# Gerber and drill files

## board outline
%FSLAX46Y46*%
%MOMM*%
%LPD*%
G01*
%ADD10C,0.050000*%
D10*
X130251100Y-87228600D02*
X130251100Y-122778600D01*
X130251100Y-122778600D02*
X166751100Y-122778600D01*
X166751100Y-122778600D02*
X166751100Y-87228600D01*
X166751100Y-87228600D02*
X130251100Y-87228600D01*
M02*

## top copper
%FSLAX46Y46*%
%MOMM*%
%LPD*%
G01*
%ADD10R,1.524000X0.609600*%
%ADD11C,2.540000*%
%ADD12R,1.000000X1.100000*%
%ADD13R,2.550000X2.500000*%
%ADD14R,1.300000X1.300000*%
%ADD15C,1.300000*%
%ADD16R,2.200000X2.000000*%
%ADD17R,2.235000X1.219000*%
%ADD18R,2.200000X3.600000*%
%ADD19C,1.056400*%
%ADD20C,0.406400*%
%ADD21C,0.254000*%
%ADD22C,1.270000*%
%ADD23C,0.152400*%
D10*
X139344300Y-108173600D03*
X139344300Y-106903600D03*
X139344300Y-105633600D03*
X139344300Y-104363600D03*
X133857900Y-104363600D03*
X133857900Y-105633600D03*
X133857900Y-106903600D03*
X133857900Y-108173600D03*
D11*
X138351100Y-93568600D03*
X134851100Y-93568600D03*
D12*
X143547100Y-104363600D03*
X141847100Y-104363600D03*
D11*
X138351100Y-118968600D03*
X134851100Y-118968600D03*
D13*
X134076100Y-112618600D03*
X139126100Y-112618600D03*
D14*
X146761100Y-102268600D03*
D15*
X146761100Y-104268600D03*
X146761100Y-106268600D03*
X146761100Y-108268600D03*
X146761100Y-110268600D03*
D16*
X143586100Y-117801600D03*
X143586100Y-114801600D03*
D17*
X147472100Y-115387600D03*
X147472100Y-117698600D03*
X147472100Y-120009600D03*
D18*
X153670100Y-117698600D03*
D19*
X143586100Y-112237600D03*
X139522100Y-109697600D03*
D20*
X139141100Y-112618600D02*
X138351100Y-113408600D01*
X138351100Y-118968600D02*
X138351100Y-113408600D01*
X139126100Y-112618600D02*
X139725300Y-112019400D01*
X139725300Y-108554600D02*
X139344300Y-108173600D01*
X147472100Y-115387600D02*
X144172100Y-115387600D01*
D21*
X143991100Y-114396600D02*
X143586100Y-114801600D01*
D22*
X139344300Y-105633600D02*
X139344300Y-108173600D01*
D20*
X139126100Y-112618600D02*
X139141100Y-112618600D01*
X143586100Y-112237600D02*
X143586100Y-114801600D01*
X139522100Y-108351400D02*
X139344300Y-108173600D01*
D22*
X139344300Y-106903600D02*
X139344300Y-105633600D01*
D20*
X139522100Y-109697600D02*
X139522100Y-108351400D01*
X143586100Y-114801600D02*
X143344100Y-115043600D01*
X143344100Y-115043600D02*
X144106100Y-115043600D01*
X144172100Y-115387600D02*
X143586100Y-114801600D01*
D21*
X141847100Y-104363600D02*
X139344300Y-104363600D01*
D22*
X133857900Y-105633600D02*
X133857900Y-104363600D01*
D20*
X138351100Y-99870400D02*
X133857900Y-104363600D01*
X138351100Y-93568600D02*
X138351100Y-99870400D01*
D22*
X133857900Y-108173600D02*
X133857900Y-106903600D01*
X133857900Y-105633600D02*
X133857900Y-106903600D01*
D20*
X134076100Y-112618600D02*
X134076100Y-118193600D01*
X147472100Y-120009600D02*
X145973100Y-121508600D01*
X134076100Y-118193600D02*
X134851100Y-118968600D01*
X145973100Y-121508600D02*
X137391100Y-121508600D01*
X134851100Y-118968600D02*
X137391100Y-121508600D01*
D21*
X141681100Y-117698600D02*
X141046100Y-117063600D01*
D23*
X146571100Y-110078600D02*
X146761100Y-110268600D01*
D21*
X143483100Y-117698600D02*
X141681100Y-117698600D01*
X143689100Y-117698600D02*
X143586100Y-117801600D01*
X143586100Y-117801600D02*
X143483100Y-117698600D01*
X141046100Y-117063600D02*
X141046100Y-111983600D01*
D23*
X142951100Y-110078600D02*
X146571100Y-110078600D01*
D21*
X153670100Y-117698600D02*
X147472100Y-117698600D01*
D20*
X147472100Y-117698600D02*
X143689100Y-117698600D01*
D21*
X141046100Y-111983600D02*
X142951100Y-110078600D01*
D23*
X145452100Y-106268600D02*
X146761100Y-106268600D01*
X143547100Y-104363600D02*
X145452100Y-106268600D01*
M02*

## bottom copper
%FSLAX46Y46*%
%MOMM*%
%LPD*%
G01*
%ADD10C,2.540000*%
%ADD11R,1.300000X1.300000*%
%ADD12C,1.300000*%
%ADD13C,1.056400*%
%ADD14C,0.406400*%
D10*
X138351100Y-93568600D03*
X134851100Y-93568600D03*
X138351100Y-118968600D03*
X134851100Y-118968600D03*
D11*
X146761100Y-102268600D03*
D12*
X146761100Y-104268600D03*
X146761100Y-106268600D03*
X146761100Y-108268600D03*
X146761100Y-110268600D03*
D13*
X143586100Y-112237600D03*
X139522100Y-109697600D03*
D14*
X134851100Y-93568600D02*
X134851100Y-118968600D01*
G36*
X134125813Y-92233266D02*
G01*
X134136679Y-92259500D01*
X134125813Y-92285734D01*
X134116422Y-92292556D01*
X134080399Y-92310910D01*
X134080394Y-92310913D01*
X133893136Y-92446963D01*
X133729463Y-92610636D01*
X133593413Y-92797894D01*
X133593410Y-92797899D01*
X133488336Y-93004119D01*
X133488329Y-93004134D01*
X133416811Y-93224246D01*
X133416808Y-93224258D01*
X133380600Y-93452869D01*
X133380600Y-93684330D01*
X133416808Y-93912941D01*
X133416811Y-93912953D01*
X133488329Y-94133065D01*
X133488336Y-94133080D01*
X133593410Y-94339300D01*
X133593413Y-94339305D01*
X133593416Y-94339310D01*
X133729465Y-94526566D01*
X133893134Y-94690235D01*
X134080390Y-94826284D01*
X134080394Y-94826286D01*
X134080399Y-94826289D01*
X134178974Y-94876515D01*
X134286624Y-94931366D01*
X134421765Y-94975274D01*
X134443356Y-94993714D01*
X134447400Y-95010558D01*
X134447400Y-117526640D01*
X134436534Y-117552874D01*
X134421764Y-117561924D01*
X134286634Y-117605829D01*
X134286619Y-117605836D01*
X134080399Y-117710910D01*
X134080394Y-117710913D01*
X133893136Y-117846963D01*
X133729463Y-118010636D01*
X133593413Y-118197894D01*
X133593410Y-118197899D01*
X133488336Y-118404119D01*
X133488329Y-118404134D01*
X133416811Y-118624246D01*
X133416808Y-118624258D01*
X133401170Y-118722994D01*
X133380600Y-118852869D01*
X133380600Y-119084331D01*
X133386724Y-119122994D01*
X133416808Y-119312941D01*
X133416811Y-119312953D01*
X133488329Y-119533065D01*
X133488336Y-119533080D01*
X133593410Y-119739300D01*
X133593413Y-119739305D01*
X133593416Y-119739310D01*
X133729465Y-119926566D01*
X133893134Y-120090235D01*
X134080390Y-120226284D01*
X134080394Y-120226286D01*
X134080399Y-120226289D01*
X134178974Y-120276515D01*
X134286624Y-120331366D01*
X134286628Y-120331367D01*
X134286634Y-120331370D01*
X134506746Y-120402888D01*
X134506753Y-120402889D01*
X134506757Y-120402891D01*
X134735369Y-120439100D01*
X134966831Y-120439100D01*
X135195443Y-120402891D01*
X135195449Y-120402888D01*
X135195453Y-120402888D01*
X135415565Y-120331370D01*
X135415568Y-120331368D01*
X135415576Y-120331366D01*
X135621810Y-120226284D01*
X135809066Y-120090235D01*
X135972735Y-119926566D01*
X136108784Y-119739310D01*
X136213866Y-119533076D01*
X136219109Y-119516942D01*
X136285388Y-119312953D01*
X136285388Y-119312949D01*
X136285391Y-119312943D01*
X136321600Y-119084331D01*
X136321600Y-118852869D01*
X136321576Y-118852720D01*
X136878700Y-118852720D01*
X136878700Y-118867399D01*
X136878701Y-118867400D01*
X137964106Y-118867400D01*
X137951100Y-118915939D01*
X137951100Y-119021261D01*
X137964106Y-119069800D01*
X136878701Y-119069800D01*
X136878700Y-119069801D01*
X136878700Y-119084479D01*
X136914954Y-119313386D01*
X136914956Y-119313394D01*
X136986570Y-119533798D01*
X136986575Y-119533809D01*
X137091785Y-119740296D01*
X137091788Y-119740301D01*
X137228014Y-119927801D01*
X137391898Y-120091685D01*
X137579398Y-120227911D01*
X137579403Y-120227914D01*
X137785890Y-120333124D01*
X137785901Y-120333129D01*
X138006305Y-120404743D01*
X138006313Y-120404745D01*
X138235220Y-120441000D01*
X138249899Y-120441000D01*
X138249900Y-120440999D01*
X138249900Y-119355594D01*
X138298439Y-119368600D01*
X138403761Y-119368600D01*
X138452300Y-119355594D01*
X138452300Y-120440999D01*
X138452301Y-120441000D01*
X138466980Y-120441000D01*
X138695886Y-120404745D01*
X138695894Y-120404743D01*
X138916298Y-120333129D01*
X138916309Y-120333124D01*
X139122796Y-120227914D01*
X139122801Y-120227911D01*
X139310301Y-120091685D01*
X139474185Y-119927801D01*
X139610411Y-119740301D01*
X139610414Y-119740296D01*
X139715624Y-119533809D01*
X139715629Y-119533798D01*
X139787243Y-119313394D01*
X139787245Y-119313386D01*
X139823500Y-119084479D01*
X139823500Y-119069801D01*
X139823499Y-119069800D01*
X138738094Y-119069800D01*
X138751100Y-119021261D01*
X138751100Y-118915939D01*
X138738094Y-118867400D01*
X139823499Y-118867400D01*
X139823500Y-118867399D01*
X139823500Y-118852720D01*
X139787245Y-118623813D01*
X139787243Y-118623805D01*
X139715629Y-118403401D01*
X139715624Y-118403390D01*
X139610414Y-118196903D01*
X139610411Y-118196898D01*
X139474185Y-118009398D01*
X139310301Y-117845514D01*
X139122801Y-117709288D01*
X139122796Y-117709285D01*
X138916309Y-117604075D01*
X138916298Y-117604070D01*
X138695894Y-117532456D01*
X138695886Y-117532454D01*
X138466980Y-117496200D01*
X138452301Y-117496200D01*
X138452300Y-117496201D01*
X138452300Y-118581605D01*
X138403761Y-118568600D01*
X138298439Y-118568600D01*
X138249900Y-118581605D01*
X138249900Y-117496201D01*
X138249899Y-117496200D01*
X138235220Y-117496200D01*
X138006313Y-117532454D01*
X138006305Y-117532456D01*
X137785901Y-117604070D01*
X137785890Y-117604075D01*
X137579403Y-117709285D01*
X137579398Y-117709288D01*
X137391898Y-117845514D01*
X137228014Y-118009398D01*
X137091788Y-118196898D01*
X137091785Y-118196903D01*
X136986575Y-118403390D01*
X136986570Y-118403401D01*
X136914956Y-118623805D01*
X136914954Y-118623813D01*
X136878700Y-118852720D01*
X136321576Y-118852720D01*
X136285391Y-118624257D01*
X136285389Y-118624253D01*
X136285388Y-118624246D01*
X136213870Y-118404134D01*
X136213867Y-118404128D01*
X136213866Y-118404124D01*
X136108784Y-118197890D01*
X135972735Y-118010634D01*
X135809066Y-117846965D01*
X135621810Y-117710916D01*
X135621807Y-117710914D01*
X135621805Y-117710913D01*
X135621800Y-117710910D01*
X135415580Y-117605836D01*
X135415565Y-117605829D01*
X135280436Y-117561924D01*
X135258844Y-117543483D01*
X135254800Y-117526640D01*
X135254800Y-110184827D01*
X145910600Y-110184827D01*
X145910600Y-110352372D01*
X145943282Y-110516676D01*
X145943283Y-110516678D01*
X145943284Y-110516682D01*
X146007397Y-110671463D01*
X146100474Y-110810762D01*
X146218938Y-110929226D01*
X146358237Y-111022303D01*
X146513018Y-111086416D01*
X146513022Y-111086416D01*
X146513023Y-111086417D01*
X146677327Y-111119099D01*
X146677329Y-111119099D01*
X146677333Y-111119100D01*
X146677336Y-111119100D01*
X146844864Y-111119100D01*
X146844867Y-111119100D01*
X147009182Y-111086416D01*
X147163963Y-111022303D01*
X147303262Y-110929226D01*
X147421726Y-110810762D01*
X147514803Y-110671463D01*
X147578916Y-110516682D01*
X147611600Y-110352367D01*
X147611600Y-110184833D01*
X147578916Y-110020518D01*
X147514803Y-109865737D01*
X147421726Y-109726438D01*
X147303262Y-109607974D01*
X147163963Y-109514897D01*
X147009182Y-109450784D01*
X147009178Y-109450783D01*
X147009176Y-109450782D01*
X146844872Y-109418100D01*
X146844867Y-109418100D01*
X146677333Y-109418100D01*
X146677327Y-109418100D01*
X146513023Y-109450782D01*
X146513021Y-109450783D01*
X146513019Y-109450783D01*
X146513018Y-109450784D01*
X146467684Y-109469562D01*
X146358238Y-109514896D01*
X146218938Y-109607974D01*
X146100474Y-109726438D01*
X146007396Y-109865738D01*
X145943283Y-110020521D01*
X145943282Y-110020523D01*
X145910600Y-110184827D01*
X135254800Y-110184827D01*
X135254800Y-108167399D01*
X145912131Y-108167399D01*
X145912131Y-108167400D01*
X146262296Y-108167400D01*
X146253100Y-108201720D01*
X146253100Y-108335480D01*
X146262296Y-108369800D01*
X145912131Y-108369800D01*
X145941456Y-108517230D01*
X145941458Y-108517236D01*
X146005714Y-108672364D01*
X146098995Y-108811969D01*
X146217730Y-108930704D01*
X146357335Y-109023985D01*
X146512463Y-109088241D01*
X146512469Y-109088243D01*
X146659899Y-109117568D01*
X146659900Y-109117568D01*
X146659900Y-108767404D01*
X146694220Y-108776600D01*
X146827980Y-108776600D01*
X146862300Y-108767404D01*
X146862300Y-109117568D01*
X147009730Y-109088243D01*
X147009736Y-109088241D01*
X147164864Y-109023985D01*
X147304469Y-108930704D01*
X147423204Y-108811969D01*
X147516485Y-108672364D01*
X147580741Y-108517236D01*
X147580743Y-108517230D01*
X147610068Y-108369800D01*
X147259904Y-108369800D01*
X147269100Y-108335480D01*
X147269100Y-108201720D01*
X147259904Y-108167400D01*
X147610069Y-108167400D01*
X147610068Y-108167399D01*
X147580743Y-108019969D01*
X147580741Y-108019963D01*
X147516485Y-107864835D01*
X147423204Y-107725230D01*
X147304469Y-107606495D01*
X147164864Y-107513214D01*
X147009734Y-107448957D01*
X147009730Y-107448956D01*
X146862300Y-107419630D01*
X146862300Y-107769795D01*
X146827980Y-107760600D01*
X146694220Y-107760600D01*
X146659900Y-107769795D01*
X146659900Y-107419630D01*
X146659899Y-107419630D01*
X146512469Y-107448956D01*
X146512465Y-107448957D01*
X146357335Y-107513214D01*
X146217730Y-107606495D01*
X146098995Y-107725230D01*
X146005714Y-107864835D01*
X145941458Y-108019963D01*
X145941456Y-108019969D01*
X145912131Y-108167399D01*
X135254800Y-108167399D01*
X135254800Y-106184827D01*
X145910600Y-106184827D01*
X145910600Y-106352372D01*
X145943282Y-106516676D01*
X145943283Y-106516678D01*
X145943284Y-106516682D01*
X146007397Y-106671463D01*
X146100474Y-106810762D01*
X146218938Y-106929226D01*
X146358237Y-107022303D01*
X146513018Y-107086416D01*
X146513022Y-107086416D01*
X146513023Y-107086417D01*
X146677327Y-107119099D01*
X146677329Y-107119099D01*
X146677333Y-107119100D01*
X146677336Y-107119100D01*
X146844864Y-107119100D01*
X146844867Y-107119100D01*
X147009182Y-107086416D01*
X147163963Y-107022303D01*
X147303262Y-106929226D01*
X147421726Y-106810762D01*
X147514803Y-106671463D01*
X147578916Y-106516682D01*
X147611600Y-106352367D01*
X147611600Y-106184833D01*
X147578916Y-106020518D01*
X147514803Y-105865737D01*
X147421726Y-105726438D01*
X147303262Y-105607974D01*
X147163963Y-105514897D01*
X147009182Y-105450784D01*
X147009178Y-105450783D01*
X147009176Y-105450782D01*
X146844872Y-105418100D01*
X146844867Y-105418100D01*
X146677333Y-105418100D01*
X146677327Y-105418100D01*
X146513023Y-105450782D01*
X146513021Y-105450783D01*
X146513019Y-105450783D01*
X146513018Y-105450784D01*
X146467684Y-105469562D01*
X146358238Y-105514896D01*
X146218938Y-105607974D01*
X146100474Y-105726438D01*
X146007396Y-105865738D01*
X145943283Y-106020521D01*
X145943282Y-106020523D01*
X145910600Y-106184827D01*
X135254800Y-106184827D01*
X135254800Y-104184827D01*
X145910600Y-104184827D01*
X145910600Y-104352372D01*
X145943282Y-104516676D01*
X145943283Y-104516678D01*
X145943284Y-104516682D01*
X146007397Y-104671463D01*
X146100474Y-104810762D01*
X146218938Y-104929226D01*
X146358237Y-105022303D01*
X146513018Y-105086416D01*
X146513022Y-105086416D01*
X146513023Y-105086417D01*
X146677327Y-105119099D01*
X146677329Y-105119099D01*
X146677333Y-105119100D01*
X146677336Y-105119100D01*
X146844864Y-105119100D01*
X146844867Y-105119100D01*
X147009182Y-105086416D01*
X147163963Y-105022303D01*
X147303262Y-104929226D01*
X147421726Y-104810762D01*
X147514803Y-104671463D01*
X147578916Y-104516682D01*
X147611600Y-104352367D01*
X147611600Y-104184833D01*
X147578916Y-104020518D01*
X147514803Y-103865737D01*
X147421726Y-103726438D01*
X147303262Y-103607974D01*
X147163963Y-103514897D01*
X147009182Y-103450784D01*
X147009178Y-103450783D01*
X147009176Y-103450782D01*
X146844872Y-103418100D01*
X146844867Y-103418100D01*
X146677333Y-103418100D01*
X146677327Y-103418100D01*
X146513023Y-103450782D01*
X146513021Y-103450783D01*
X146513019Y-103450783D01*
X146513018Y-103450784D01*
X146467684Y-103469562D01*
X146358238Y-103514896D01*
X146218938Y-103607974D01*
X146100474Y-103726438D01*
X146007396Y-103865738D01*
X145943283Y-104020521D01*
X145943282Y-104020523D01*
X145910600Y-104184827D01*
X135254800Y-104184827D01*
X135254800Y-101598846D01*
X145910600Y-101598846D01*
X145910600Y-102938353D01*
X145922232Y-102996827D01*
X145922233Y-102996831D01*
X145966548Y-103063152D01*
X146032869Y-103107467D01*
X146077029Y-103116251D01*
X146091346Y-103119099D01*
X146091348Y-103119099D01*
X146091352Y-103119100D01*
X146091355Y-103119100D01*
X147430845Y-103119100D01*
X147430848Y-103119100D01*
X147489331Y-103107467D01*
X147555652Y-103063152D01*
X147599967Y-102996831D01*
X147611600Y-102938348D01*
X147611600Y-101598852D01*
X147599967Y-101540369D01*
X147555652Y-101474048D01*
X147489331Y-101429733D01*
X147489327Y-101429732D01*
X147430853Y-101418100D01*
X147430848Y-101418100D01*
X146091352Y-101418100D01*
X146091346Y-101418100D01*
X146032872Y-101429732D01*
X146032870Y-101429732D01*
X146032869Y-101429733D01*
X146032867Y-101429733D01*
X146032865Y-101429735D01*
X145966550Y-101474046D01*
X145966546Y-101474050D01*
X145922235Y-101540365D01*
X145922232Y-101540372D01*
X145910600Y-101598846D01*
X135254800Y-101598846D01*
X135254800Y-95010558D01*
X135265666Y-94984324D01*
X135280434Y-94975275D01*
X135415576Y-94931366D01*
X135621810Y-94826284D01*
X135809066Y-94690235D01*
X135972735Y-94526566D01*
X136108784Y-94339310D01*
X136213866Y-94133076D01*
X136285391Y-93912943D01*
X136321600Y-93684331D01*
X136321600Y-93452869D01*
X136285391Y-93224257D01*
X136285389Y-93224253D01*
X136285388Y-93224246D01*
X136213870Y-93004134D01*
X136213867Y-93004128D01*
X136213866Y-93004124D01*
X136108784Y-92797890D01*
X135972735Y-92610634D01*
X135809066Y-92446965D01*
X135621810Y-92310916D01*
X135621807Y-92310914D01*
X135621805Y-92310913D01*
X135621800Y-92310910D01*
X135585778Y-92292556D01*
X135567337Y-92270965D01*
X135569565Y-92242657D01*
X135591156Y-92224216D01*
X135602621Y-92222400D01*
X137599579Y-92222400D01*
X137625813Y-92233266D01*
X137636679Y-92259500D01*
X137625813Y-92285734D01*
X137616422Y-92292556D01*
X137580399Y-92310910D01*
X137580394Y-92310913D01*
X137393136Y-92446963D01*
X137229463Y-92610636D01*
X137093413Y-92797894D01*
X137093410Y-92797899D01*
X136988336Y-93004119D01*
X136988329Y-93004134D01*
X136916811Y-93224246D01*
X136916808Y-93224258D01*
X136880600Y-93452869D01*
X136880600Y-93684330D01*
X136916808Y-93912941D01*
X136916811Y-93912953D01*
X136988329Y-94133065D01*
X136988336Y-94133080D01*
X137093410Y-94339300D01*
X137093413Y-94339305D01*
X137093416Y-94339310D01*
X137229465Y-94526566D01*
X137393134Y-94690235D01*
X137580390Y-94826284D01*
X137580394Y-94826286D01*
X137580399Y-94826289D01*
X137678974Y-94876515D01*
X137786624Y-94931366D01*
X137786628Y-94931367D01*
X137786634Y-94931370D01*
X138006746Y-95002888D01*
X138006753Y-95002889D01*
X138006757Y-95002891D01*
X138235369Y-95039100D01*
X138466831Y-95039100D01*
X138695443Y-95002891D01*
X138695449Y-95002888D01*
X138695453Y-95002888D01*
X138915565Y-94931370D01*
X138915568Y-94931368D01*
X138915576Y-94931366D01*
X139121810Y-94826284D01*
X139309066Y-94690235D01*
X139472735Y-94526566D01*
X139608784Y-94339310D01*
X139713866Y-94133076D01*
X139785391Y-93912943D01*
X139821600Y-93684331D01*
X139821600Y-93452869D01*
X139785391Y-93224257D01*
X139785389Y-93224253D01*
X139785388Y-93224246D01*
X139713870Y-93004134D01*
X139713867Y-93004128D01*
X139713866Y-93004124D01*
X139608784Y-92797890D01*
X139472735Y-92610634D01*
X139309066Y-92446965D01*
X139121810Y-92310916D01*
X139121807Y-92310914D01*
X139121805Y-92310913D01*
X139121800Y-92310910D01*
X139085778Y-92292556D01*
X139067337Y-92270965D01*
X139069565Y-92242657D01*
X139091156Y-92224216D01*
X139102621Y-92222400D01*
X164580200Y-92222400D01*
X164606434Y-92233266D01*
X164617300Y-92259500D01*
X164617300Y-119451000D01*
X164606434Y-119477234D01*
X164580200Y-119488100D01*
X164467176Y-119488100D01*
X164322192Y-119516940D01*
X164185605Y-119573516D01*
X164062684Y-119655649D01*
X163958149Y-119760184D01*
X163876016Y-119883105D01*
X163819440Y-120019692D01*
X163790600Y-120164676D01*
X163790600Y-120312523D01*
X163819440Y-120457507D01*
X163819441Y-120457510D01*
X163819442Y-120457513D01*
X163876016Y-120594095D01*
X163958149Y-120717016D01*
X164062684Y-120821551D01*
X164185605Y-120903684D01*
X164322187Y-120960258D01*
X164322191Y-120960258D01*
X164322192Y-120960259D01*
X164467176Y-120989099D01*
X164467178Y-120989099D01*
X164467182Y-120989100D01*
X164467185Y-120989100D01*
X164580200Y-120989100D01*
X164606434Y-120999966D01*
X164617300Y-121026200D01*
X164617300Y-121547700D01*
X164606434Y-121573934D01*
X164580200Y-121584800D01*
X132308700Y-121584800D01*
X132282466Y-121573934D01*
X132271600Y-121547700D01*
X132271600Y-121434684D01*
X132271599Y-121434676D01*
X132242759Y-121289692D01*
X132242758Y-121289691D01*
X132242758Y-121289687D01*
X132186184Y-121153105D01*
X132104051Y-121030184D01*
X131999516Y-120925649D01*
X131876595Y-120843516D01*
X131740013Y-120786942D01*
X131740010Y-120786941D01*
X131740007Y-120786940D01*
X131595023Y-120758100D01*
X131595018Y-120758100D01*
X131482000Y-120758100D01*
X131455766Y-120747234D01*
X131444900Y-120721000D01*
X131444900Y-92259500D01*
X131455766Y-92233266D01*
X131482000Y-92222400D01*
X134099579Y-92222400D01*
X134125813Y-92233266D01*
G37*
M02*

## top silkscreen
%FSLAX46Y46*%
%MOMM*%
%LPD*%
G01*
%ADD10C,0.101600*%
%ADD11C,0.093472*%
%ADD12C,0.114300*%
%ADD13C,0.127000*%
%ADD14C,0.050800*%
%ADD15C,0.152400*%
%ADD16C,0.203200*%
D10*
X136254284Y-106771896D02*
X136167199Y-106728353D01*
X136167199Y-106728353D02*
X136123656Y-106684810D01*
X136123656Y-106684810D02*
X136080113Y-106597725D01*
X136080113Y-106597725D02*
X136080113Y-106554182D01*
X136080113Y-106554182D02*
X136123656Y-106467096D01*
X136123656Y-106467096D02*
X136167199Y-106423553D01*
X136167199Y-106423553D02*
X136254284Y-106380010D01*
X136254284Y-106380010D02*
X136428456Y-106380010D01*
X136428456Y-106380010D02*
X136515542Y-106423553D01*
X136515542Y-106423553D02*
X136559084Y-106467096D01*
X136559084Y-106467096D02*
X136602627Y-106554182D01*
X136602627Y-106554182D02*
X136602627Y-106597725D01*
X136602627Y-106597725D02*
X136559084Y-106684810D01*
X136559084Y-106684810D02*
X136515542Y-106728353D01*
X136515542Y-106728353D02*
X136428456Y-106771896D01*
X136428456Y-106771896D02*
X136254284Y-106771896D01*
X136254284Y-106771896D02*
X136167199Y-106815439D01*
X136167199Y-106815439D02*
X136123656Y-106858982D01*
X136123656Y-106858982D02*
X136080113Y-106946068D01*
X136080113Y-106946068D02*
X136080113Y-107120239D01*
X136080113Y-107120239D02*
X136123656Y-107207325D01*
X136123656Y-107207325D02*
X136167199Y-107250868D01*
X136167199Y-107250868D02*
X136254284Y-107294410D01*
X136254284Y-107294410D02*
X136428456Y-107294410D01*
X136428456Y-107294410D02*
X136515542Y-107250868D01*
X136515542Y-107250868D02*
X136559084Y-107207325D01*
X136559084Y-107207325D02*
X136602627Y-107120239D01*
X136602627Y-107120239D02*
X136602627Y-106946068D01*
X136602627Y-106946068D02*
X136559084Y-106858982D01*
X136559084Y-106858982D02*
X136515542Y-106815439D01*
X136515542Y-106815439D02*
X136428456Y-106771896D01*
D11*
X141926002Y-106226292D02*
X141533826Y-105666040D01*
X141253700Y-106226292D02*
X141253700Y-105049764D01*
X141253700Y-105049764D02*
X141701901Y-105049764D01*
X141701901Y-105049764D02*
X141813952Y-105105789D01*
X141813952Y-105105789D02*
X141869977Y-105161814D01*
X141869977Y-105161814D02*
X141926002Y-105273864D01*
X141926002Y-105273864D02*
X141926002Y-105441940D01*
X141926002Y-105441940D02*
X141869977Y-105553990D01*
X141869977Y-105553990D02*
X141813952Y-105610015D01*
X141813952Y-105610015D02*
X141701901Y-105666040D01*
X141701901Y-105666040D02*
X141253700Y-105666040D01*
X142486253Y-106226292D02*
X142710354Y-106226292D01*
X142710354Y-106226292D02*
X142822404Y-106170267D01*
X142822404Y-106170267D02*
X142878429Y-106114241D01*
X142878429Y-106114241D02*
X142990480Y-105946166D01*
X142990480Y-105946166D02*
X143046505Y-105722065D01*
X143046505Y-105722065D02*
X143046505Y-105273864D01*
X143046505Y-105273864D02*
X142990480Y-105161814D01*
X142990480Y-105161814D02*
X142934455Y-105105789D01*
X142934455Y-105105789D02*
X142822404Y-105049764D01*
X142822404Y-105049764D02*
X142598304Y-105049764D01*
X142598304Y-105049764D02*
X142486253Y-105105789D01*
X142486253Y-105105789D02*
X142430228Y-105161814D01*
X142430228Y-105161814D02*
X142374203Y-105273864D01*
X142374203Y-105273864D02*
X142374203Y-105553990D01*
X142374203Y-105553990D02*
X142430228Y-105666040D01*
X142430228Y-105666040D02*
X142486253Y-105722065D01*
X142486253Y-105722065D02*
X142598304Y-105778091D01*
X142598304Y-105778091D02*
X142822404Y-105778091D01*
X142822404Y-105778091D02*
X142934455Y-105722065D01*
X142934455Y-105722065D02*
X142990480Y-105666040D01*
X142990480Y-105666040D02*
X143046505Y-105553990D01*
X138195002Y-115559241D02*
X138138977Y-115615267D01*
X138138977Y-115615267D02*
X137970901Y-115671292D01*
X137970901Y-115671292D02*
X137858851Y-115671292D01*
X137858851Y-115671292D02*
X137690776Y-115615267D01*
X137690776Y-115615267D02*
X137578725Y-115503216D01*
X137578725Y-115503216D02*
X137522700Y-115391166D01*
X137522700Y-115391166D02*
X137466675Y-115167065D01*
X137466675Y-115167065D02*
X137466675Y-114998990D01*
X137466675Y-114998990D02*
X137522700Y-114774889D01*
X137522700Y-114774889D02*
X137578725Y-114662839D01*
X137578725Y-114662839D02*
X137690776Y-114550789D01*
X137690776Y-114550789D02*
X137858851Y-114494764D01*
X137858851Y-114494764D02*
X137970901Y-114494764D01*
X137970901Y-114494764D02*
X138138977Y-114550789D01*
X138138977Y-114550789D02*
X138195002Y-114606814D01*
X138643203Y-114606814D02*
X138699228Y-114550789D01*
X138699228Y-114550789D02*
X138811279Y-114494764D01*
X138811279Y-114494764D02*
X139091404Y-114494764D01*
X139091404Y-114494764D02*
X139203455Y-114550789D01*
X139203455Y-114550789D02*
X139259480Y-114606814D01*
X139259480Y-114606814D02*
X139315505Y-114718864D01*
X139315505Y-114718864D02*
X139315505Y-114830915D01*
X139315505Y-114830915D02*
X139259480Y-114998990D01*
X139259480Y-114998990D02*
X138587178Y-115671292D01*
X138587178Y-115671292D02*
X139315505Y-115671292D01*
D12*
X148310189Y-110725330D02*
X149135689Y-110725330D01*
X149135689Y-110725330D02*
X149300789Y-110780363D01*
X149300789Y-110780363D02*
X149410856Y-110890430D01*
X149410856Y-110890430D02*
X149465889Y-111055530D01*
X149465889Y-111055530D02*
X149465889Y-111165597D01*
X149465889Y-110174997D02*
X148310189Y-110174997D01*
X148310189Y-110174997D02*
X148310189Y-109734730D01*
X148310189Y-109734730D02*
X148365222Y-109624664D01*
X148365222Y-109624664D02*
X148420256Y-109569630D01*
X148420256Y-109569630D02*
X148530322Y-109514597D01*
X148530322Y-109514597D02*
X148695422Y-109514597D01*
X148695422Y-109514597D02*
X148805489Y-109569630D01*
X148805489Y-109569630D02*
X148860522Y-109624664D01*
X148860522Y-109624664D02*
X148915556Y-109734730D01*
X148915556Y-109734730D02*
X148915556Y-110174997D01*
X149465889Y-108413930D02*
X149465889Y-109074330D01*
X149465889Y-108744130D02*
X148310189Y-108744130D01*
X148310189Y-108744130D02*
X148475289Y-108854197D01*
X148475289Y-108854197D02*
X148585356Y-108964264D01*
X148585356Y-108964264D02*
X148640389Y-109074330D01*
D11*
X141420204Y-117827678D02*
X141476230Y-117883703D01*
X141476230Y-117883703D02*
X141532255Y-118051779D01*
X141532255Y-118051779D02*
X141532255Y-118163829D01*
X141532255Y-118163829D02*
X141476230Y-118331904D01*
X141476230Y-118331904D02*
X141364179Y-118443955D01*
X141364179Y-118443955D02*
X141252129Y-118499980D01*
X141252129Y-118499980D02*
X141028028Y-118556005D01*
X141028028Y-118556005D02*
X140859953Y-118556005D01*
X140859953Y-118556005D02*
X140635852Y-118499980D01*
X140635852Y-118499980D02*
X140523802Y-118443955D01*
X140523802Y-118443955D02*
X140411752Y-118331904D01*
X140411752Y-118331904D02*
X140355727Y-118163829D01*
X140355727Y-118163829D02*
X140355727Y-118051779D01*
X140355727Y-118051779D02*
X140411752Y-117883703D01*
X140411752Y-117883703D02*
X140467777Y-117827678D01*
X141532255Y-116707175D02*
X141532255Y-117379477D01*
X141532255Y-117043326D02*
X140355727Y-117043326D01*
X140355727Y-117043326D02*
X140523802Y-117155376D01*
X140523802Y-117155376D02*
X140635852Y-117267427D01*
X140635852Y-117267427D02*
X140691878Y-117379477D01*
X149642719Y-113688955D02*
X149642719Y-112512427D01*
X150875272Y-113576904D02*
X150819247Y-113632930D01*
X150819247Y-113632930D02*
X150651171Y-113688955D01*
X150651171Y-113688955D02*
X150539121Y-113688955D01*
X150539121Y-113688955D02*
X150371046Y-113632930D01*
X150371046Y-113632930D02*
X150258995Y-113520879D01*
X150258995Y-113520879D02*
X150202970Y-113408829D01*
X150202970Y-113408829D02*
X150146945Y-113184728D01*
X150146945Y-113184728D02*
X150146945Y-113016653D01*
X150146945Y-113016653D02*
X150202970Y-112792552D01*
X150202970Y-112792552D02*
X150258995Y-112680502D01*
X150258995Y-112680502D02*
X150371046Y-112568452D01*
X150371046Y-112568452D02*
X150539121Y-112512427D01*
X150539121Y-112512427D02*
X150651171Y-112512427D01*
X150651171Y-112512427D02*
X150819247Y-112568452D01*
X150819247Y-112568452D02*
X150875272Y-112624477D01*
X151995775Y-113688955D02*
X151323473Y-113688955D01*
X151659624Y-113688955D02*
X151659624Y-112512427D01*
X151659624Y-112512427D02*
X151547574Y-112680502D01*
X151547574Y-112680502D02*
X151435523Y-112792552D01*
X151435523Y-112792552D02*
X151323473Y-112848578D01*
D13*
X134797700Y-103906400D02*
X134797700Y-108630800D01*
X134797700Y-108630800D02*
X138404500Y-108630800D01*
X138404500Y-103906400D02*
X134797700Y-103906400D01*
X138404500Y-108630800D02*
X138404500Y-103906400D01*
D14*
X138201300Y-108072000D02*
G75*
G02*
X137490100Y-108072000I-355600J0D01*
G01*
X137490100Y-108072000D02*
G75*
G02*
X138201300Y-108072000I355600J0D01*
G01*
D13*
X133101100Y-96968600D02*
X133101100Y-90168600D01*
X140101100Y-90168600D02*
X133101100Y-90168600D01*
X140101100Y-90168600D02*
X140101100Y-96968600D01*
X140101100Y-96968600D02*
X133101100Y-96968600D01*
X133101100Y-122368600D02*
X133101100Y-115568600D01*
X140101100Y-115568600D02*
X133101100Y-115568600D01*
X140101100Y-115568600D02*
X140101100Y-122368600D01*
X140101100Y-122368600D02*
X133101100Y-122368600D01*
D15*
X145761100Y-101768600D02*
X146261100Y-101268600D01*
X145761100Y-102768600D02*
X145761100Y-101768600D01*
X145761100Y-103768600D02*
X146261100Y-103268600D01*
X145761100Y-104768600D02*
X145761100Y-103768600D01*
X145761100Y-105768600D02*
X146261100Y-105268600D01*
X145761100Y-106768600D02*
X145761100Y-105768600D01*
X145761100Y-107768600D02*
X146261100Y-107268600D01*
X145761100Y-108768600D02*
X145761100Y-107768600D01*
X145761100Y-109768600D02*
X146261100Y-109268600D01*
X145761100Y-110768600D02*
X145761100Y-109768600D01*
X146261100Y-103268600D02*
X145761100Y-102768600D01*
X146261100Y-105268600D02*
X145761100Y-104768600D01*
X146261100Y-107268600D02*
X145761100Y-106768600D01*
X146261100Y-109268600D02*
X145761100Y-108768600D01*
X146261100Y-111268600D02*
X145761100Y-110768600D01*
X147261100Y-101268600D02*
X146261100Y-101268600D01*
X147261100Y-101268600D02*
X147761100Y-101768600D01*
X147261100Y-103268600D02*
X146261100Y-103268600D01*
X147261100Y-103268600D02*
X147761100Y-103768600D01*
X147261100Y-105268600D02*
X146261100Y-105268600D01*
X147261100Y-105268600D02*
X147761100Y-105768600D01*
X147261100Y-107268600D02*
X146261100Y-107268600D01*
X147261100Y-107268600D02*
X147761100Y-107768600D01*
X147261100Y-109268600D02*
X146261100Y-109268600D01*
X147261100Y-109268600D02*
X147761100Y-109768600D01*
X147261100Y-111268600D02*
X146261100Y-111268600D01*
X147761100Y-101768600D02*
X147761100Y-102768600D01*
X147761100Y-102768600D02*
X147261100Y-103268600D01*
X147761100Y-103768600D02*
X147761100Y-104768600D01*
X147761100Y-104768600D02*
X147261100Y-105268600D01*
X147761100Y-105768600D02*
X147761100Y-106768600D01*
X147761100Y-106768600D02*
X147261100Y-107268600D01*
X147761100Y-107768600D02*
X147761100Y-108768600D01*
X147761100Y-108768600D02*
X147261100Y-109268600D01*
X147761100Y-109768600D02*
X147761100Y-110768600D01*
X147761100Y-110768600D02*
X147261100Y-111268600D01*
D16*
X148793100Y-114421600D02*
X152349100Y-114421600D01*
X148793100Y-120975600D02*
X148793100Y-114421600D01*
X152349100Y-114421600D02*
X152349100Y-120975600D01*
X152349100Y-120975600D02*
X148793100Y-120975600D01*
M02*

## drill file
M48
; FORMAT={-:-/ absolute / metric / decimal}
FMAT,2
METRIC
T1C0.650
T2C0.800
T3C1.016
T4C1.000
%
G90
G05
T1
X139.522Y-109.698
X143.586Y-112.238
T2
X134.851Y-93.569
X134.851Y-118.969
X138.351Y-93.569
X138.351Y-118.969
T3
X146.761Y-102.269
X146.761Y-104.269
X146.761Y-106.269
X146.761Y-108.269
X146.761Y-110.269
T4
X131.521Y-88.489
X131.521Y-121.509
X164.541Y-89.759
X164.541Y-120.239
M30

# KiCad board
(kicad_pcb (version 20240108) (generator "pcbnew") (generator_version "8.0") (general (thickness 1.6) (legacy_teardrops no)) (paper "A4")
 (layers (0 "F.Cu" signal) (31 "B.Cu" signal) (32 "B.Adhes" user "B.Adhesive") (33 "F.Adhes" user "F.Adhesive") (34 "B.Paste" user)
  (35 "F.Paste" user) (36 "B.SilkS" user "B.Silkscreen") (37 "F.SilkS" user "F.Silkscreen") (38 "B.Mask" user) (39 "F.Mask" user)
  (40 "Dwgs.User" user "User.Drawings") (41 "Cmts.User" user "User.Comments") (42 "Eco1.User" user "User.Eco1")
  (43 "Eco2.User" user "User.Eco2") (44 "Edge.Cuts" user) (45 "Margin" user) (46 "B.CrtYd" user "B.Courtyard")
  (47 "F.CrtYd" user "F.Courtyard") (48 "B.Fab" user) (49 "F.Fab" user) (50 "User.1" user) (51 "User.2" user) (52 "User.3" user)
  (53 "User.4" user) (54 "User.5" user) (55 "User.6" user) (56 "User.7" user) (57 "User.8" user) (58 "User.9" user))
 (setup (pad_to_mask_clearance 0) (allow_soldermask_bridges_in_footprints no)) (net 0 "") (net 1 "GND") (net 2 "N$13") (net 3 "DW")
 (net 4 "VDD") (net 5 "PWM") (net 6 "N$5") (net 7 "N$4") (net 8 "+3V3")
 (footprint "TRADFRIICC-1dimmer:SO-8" (layer "F.Cu") (at 136.6011 106.2686 180)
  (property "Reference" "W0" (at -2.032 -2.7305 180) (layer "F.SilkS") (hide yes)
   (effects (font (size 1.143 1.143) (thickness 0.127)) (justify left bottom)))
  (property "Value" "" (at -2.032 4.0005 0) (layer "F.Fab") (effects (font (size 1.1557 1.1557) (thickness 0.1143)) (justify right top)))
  (fp_line (start 1.8034 2.3622) (end 1.8034 -2.3622) (stroke (width 0.127) (type solid)) (layer "F.SilkS"))
  (fp_line (start 1.8034 -2.3622) (end -1.8034 -2.3622) (stroke (width 0.127) (type solid)) (layer "F.SilkS"))
  (fp_line (start -1.8034 2.3622) (end 1.8034 2.3622) (stroke (width 0.127) (type solid)) (layer "F.SilkS"))
  (fp_line (start -1.8034 -2.3622) (end -1.8034 2.3622) (stroke (width 0.127) (type solid)) (layer "F.SilkS"))
  (fp_circle (center -1.2446 -1.8034) (end -0.889 -1.8034) (stroke (width 0.0508) (type solid)) (fill none) (layer "F.SilkS"))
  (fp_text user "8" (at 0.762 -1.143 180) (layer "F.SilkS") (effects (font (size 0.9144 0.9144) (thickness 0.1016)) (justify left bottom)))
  (pad "1" smd rect (at -2.7432 -1.905 180) (size 1.524 0.6096) (layers "F.Cu" "F.Paste" "F.Mask") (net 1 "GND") (solder_mask_margin 0.1016)
   (thermal_bridge_angle 0))
  (pad "2" smd rect (at -2.7432 -0.635 180) (size 1.524 0.6096) (layers "F.Cu" "F.Paste" "F.Mask") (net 1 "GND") (solder_mask_margin 0.1016)
   (thermal_bridge_angle 0))
  (pad "3" smd rect (at -2.7432 0.635 180) (size 1.524 0.6096) (layers "F.Cu" "F.Paste" "F.Mask") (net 1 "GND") (solder_mask_margin 0.1016)
   (thermal_bridge_angle 0))
  (pad "4" smd rect (at -2.7432 1.905 180) (size 1.524 0.6096) (layers "F.Cu" "F.Paste" "F.Mask") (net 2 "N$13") (solder_mask_margin 0.1016)
   (thermal_bridge_angle 0))
  (pad "5" smd rect (at 2.7432 1.905 180) (size 1.524 0.6096) (layers "F.Cu" "F.Paste" "F.Mask") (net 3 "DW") (solder_mask_margin 0.1016)
   (thermal_bridge_angle 0))
  (pad "6" smd rect (at 2.7432 0.635 180) (size 1.524 0.6096) (layers "F.Cu" "F.Paste" "F.Mask") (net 3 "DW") (solder_mask_margin 0.1016)
   (thermal_bridge_angle 0))
  (pad "7" smd rect (at 2.7432 -0.635 180) (size 1.524 0.6096) (layers "F.Cu" "F.Paste" "F.Mask") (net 3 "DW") (solder_mask_margin 0.1016)
   (thermal_bridge_angle 0))
  (pad "8" smd rect (at 2.7432 -1.905 180) (size 1.524 0.6096) (layers "F.Cu" "F.Paste" "F.Mask") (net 3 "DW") (solder_mask_margin 0.1016)
   (thermal_bridge_angle 0)))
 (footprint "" (layer "F.Cu") (at 164.5411 89.7586)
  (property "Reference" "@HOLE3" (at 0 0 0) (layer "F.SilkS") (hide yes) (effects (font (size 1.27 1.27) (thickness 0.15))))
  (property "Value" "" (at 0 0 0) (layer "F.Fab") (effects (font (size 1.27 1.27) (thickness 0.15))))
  (pad "" np_thru_hole circle (at 0 0) (size 1 1) (drill 1) (layers "*.Cu" "*.Mask")))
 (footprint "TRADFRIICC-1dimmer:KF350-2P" (layer "F.Cu") (at 136.6011 93.5686 180)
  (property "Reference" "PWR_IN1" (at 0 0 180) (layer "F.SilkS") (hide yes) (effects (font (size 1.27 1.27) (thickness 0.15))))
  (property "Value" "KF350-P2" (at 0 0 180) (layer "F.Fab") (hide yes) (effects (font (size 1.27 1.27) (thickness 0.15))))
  (fp_line (start 3.5 -3.4) (end 3.5 3.4) (stroke (width 0.127) (type solid)) (layer "F.SilkS"))
  (fp_line (start -3.5 3.4) (end 3.5 3.4) (stroke (width 0.127) (type solid)) (layer "F.SilkS"))
  (fp_line (start -3.5 3.4) (end -3.5 -3.4) (stroke (width 0.127) (type solid)) (layer "F.SilkS"))
  (fp_line (start -3.5 -3.4) (end 3.5 -3.4) (stroke (width 0.127) (type solid)) (layer "F.SilkS"))
  (pad "1" thru_hole circle (at -1.75 0 180) (size 2.54 2.54) (drill 0.8) (layers "*.Cu" "*.Mask") (remove_unused_layers no) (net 3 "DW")
   (solder_mask_margin 0.1016) (thermal_bridge_angle 0))
  (pad "2" thru_hole circle (at 1.75 0 180) (size 2.54 2.54) (drill 0.8) (layers "*.Cu" "*.Mask") (remove_unused_layers no) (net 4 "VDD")
   (solder_mask_margin 0.1016) (thermal_bridge_angle 0)))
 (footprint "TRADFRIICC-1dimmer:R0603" (layer "F.Cu") (at 142.6971 104.3636 180)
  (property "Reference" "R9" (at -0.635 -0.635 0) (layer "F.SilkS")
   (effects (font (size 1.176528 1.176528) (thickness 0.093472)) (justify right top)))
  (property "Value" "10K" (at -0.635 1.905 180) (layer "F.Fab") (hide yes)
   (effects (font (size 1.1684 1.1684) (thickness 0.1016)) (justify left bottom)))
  (pad "1" smd rect (at -0.85 0 180) (size 1 1.1) (layers "F.Cu" "F.Paste" "F.Mask") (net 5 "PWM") (solder_mask_margin 0.1016)
   (thermal_bridge_angle 0))
  (pad "2" smd rect (at 0.85 0 180) (size 1 1.1) (layers "F.Cu" "F.Paste" "F.Mask") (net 2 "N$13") (solder_mask_margin 0.1016)
   (thermal_bridge_angle 0)))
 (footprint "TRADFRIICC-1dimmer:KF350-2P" (layer "F.Cu") (at 136.6011 118.9686 180)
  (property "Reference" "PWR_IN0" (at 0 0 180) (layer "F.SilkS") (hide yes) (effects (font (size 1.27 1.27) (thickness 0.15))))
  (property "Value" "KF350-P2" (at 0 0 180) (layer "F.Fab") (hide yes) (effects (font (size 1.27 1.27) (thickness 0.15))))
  (fp_line (start 3.5 -3.4) (end 3.5 3.4) (stroke (width 0.127) (type solid)) (layer "F.SilkS"))
  (fp_line (start -3.5 3.4) (end 3.5 3.4) (stroke (width 0.127) (type solid)) (layer "F.SilkS"))
  (fp_line (start -3.5 3.4) (end -3.5 -3.4) (stroke (width 0.127) (type solid)) (layer "F.SilkS"))
  (fp_line (start -3.5 -3.4) (end 3.5 -3.4) (stroke (width 0.127) (type solid)) (layer "F.SilkS"))
  (pad "1" thru_hole circle (at -1.75 0 180) (size 2.54 2.54) (drill 0.8) (layers "*.Cu" "*.Mask") (remove_unused_layers no) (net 1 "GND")
   (solder_mask_margin 0.1016) (thermal_bridge_angle 0))
  (pad "2" thru_hole circle (at 1.75 0 180) (size 2.54 2.54) (drill 0.8) (layers "*.Cu" "*.Mask") (remove_unused_layers no) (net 4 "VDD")
   (solder_mask_margin 0.1016) (thermal_bridge_angle 0)))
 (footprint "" (layer "F.Cu") (at 131.5211 121.5086)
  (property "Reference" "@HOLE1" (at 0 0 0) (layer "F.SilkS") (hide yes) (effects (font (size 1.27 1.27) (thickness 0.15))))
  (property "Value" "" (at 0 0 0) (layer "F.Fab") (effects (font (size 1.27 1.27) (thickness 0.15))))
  (pad "" np_thru_hole circle (at 0 0) (size 1 1) (drill 1) (layers "*.Cu" "*.Mask")))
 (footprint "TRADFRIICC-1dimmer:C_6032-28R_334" (layer "F.Cu") (at 136.6011 112.6186 180)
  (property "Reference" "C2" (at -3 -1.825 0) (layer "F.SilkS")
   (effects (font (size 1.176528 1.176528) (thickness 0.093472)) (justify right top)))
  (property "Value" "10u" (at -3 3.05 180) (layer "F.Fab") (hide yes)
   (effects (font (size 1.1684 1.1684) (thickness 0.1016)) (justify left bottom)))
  (pad "+" smd rect (at 2.525 0 180) (size 2.55 2.5) (layers "F.Cu" "F.Paste" "F.Mask") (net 4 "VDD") (solder_mask_margin 0.1016)
   (thermal_bridge_angle 0))
  (pad "-" smd rect (at -2.525 0 180) (size 2.55 2.5) (layers "F.Cu" "F.Paste" "F.Mask") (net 1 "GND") (solder_mask_margin 0.1016)
   (thermal_bridge_angle 0)))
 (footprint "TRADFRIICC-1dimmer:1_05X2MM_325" (layer "F.Cu") (at 146.7611 106.2686 -90)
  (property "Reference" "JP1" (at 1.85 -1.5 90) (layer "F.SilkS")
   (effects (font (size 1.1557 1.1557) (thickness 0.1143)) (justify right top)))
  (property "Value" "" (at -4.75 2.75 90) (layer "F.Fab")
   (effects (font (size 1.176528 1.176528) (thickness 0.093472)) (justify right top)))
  (fp_line (start -4.5 1) (end -5 0.5) (stroke (width 0.1524) (type solid)) (layer "F.SilkS"))
  (fp_line (start -3.5 1) (end -4.5 1) (stroke (width 0.1524) (type solid)) (layer "F.SilkS"))
  (fp_line (start -2.5 1) (end -3 0.5) (stroke (width 0.1524) (type solid)) (layer "F.SilkS"))
  (fp_line (start -1.5 1) (end -2.5 1) (stroke (width 0.1524) (type solid)) (layer "F.SilkS"))
  (fp_line (start -0.5 1) (end -1 0.5) (stroke (width 0.1524) (type solid)) (layer "F.SilkS"))
  (fp_line (start 0.5 1) (end -0.5 1) (stroke (width 0.1524) (type solid)) (layer "F.SilkS"))
  (fp_line (start 1.5 1) (end 1 0.5) (stroke (width 0.1524) (type solid)) (layer "F.SilkS"))
  (fp_line (start 2.5 1) (end 1.5 1) (stroke (width 0.1524) (type solid)) (layer "F.SilkS"))
  (fp_line (start 3.5 1) (end 3 0.5) (stroke (width 0.1524) (type solid)) (layer "F.SilkS"))
  (fp_line (start 4.5 1) (end 3.5 1) (stroke (width 0.1524) (type solid)) (layer "F.SilkS"))
  (fp_line (start -3 0.5) (end -3.5 1) (stroke (width 0.1524) (type solid)) (layer "F.SilkS"))
  (fp_line (start -1 0.5) (end -1.5 1) (stroke (width 0.1524) (type solid)) (layer "F.SilkS"))
  (fp_line (start 1 0.5) (end 0.5 1) (stroke (width 0.1524) (type solid)) (layer "F.SilkS"))
  (fp_line (start 3 0.5) (end 2.5 1) (stroke (width 0.1524) (type solid)) (layer "F.SilkS"))
  (fp_line (start 5 0.5) (end 4.5 1) (stroke (width 0.1524) (type solid)) (layer "F.SilkS"))
  (fp_line (start -5 -0.5) (end -5 0.5) (stroke (width 0.1524) (type solid)) (layer "F.SilkS"))
  (fp_line (start -5 -0.5) (end -4.5 -1) (stroke (width 0.1524) (type solid)) (layer "F.SilkS"))
  (fp_line (start -3 -0.5) (end -3 0.5) (stroke (width 0.1524) (type solid)) (layer "F.SilkS"))
  (fp_line (start -3 -0.5) (end -2.5 -1) (stroke (width 0.1524) (type solid)) (layer "F.SilkS"))
  (fp_line (start -1 -0.5) (end -1 0.5) (stroke (width 0.1524) (type solid)) (layer "F.SilkS"))
  (fp_line (start -1 -0.5) (end -0.5 -1) (stroke (width 0.1524) (type solid)) (layer "F.SilkS"))
  (fp_line (start 1 -0.5) (end 1 0.5) (stroke (width 0.1524) (type solid)) (layer "F.SilkS"))
  (fp_line (start 1 -0.5) (end 1.5 -1) (stroke (width 0.1524) (type solid)) (layer "F.SilkS"))
  (fp_line (start 3 -0.5) (end 3 0.5) (stroke (width 0.1524) (type solid)) (layer "F.SilkS"))
  (fp_line (start 3 -0.5) (end 3.5 -1) (stroke (width 0.1524) (type solid)) (layer "F.SilkS"))
  (fp_line (start 5 -0.5) (end 5 0.5) (stroke (width 0.1524) (type solid)) (layer "F.SilkS"))
  (fp_line (start -4.5 -1) (end -3.5 -1) (stroke (width 0.1524) (type solid)) (layer "F.SilkS"))
  (fp_line (start -3.5 -1) (end -3 -0.5) (stroke (width 0.1524) (type solid)) (layer "F.SilkS"))
  (fp_line (start -2.5 -1) (end -1.5 -1) (stroke (width 0.1524) (type solid)) (layer "F.SilkS"))
  (fp_line (start -1.5 -1) (end -1 -0.5) (stroke (width 0.1524) (type solid)) (layer "F.SilkS"))
  (fp_line (start -0.5 -1) (end 0.5 -1) (stroke (width 0.1524) (type solid)) (layer "F.SilkS"))
  (fp_line (start 0.5 -1) (end 1 -0.5) (stroke (width 0.1524) (type solid)) (layer "F.SilkS"))
  (fp_line (start 1.5 -1) (end 2.5 -1) (stroke (width 0.1524) (type solid)) (layer "F.SilkS"))
  (fp_line (start 2.5 -1) (end 3 -0.5) (stroke (width 0.1524) (type solid)) (layer "F.SilkS"))
  (fp_line (start 3.5 -1) (end 4.5 -1) (stroke (width 0.1524) (type solid)) (layer "F.SilkS"))
  (fp_line (start 4.5 -1) (end 5 -0.5) (stroke (width 0.1524) (type solid)) (layer "F.SilkS"))
  (pad "1" thru_hole rect (at -4 0) (size 1.3 1.3) (drill 1.016) (layers "*.Cu" "*.Mask") (remove_unused_layers no) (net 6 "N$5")
   (solder_mask_margin 0.1016) (thermal_bridge_angle 0))
  (pad "2" thru_hole circle (at -2 0) (size 1.3 1.3) (drill 1.016) (layers "*.Cu" "*.Mask") (remove_unused_layers no) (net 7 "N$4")
   (solder_mask_margin 0.1016) (thermal_bridge_angle 0))
  (pad "3" thru_hole circle (at 0 0) (size 1.3 1.3) (drill 1.016) (layers "*.Cu" "*.Mask") (remove_unused_layers no) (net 5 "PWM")
   (solder_mask_margin 0.1016) (thermal_bridge_angle 0))
  (pad "4" thru_hole circle (at 2 0) (size 1.3 1.3) (drill 1.016) (layers "*.Cu" "*.Mask") (remove_unused_layers no) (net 1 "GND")
   (solder_mask_margin 0.1016) (thermal_bridge_angle 0))
  (pad "5" thru_hole circle (at 4 0) (size 1.3 1.3) (drill 1.016) (layers "*.Cu" "*.Mask") (remove_unused_layers no) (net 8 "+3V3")
   (solder_mask_margin 0.1016) (thermal_bridge_angle 0)))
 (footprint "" (layer "F.Cu") (at 131.5211 88.4886)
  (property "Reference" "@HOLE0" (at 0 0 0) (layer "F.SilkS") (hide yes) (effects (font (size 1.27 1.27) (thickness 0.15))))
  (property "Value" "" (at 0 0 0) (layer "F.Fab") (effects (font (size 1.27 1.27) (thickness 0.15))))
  (pad "" np_thru_hole circle (at 0 0) (size 1 1) (drill 1) (layers "*.Cu" "*.Mask")))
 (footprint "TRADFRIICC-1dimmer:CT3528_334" (layer "F.Cu") (at 143.5861 116.3016 90)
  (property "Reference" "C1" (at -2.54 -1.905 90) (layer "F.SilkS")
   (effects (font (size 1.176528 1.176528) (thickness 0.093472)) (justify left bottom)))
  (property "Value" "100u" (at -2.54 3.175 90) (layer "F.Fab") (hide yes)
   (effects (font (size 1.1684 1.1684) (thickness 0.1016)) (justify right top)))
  (pad "+" smd rect (at -1.5 0 90) (size 2 2.2) (layers "F.Cu" "F.Paste" "F.Mask") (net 8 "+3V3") (solder_mask_margin 0.1016)
   (thermal_bridge_angle 0))
  (pad "-" smd rect (at 1.5 0 90) (size 2 2.2) (layers "F.Cu" "F.Paste" "F.Mask") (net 1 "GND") (solder_mask_margin 0.1016)
   (thermal_bridge_angle 0)))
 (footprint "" (layer "F.Cu") (at 164.5411 120.2386)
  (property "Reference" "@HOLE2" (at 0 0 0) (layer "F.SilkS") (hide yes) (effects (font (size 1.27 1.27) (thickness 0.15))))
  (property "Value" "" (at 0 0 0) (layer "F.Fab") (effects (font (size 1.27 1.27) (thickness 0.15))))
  (pad "" np_thru_hole circle (at 0 0) (size 1 1) (drill 1) (layers "*.Cu" "*.Mask")))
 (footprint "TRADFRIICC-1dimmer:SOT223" (layer "F.Cu") (at 150.5711 117.6986 -90)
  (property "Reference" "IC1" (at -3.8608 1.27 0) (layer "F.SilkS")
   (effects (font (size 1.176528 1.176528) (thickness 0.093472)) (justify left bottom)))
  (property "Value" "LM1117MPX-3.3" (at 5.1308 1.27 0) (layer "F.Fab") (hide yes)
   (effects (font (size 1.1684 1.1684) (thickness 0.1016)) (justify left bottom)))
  (fp_line (start -3.277 1.778) (end -3.277 -1.778) (stroke (width 0.2032) (type solid)) (layer "F.SilkS"))
  (fp_line (start 3.277 1.778) (end -3.277 1.778) (stroke (width 0.2032) (type solid)) (layer "F.SilkS"))
  (fp_line (start -3.277 -1.778) (end 3.277 -1.778) (stroke (width 0.2032) (type solid)) (layer "F.SilkS"))
  (fp_line (start 3.277 -1.778) (end 3.277 1.778) (stroke (width 0.2032) (type solid)) (layer "F.SilkS"))
  (pad "1" smd rect (at -2.311 3.099 270) (size 1.219 2.235) (layers "F.Cu" "F.Paste" "F.Mask") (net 1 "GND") (solder_mask_margin 0.1016)
   (thermal_bridge_angle 0))
  (pad "2" smd rect (at 0 3.099 270) (size 1.219 2.235) (layers "F.Cu" "F.Paste" "F.Mask") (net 8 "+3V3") (solder_mask_margin 0.1016)
   (thermal_bridge_angle 0))
  (pad "3" smd rect (at 2.311 3.099 270) (size 1.219 2.235) (layers "F.Cu" "F.Paste" "F.Mask") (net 4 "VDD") (solder_mask_margin 0.1016)
   (thermal_bridge_angle 0))
  (pad "TAB" smd rect (at 0 -3.099 270) (size 3.6 2.2) (layers "F.Cu" "F.Paste" "F.Mask") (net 8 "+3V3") (solder_mask_margin 0.1016)
   (thermal_bridge_angle 0)))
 (gr_line (start 130.2511 87.2286) (end 130.2511 122.7786) (stroke (width 0.05) (type solid)) (layer "Edge.Cuts"))
 (gr_line (start 130.2511 122.7786) (end 166.7511 122.7786) (stroke (width 0.05) (type solid)) (layer "Edge.Cuts"))
 (gr_line (start 166.7511 122.7786) (end 166.7511 87.2286) (stroke (width 0.05) (type solid)) (layer "Edge.Cuts"))
 (gr_line (start 166.7511 87.2286) (end 130.2511 87.2286) (stroke (width 0.05) (type solid)) (layer "Edge.Cuts"))
 (segment (start 139.1411 112.6186) (end 138.3511 113.4086) (width 0.4064) (layer "F.Cu") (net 1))
 (segment (start 138.3511 118.9686) (end 138.3511 113.4086) (width 0.4064) (layer "F.Cu") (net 1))
 (segment (start 139.1261 112.6186) (end 139.7253 112.0194) (width 0.4064) (layer "F.Cu") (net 1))
 (segment (start 139.7253 108.5546) (end 139.3443 108.1736) (width 0.4064) (layer "F.Cu") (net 1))
 (segment (start 147.4721 115.3876) (end 144.1721 115.3876) (width 0.4064) (layer "F.Cu") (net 1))
 (segment (start 143.9911 114.3966) (end 143.5861 114.8016) (width 0.254) (layer "F.Cu") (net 1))
 (segment (start 139.3443 105.6336) (end 139.3443 108.1736) (width 1.27) (layer "F.Cu") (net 1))
 (segment (start 139.1261 112.6186) (end 139.1411 112.6186) (width 0.4064) (layer "F.Cu") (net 1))
 (segment (start 143.5861 112.2376) (end 143.5861 114.8016) (width 0.4064) (layer "F.Cu") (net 1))
 (segment (start 139.5221 108.3514) (end 139.3443 108.1736) (width 0.4064) (layer "F.Cu") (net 1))
 (segment (start 139.3443 106.9036) (end 139.3443 105.6336) (width 1.27) (layer "F.Cu") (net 1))
 (segment (start 139.5221 109.6976) (end 139.5221 108.3514) (width 0.4064) (layer "F.Cu") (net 1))
 (segment (start 143.5861 114.8016) (end 143.3441 115.0436) (width 0.4064) (layer "F.Cu") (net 1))
 (segment (start 143.3441 115.0436) (end 144.1061 115.0436) (width 0.4064) (layer "F.Cu") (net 1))
 (segment (start 144.1721 115.3876) (end 143.5861 114.8016) (width 0.4064) (layer "F.Cu") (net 1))
 (via (at 143.5861 112.2376) (size 1.0564) (drill 0.65) (layers "F.Cu" "B.Cu") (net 1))
 (via (at 139.5221 109.6976) (size 1.0564) (drill 0.65) (layers "F.Cu" "B.Cu") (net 1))
 (segment (start 141.8471 104.3636) (end 139.3443 104.3636) (width 0.254) (layer "F.Cu") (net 2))
 (segment (start 133.8579 105.6336) (end 133.8579 104.3636) (width 1.27) (layer "F.Cu") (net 3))
 (segment (start 138.3511 99.8704) (end 133.8579 104.3636) (width 0.4064) (layer "F.Cu") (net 3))
 (segment (start 138.3511 93.5686) (end 138.3511 99.8704) (width 0.4064) (layer "F.Cu") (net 3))
 (segment (start 133.8579 108.1736) (end 133.8579 106.9036) (width 1.27) (layer "F.Cu") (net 3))
 (segment (start 133.8579 105.6336) (end 133.8579 106.9036) (width 1.27) (layer "F.Cu") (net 3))
 (segment (start 134.0761 112.6186) (end 134.0761 118.1936) (width 0.4064) (layer "F.Cu") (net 4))
 (segment (start 147.4721 120.0096) (end 145.9731 121.5086) (width 0.4064) (layer "F.Cu") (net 4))
 (segment (start 134.0761 118.1936) (end 134.8511 118.9686) (width 0.4064) (layer "F.Cu") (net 4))
 (segment (start 145.9731 121.5086) (end 137.3911 121.5086) (width 0.4064) (layer "F.Cu") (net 4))
 (segment (start 134.8511 118.9686) (end 137.3911 121.5086) (width 0.4064) (layer "F.Cu") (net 4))
 (segment (start 134.8511 93.5686) (end 134.8511 118.9686) (width 0.4064) (layer "B.Cu") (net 4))
 (segment (start 141.6811 117.6986) (end 141.0461 117.0636) (width 0.254) (layer "F.Cu") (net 8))
 (segment (start 146.5711 110.0786) (end 146.7611 110.2686) (width 0.1524) (layer "F.Cu") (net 8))
 (segment (start 143.4831 117.6986) (end 141.6811 117.6986) (width 0.254) (layer "F.Cu") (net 8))
 (segment (start 143.6891 117.6986) (end 143.5861 117.8016) (width 0.254) (layer "F.Cu") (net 8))
 (segment (start 143.5861 117.8016) (end 143.4831 117.6986) (width 0.254) (layer "F.Cu") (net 8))
 (segment (start 141.0461 117.0636) (end 141.0461 111.9836) (width 0.254) (layer "F.Cu") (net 8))
 (segment (start 142.9511 110.0786) (end 146.5711 110.0786) (width 0.1524) (layer "F.Cu") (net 8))
 (segment (start 153.6701 117.6986) (end 147.4721 117.6986) (width 0.254) (layer "F.Cu") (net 8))
 (segment (start 147.4721 117.6986) (end 143.6891 117.6986) (width 0.4064) (layer "F.Cu") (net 8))
 (segment (start 141.0461 111.9836) (end 142.9511 110.0786) (width 0.254) (layer "F.Cu") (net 8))
 (segment (start 145.4521 106.2686) (end 146.7611 106.2686) (width 0.1524) (layer "F.Cu") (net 5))
 (segment (start 143.5471 104.3636) (end 145.4521 106.2686) (width 0.1524) (layer "F.Cu") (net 5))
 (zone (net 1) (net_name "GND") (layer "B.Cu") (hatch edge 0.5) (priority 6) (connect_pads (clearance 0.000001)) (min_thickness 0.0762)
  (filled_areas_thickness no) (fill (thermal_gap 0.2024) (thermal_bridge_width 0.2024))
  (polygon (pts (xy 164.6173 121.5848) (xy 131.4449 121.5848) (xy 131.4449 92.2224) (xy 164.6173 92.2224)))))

